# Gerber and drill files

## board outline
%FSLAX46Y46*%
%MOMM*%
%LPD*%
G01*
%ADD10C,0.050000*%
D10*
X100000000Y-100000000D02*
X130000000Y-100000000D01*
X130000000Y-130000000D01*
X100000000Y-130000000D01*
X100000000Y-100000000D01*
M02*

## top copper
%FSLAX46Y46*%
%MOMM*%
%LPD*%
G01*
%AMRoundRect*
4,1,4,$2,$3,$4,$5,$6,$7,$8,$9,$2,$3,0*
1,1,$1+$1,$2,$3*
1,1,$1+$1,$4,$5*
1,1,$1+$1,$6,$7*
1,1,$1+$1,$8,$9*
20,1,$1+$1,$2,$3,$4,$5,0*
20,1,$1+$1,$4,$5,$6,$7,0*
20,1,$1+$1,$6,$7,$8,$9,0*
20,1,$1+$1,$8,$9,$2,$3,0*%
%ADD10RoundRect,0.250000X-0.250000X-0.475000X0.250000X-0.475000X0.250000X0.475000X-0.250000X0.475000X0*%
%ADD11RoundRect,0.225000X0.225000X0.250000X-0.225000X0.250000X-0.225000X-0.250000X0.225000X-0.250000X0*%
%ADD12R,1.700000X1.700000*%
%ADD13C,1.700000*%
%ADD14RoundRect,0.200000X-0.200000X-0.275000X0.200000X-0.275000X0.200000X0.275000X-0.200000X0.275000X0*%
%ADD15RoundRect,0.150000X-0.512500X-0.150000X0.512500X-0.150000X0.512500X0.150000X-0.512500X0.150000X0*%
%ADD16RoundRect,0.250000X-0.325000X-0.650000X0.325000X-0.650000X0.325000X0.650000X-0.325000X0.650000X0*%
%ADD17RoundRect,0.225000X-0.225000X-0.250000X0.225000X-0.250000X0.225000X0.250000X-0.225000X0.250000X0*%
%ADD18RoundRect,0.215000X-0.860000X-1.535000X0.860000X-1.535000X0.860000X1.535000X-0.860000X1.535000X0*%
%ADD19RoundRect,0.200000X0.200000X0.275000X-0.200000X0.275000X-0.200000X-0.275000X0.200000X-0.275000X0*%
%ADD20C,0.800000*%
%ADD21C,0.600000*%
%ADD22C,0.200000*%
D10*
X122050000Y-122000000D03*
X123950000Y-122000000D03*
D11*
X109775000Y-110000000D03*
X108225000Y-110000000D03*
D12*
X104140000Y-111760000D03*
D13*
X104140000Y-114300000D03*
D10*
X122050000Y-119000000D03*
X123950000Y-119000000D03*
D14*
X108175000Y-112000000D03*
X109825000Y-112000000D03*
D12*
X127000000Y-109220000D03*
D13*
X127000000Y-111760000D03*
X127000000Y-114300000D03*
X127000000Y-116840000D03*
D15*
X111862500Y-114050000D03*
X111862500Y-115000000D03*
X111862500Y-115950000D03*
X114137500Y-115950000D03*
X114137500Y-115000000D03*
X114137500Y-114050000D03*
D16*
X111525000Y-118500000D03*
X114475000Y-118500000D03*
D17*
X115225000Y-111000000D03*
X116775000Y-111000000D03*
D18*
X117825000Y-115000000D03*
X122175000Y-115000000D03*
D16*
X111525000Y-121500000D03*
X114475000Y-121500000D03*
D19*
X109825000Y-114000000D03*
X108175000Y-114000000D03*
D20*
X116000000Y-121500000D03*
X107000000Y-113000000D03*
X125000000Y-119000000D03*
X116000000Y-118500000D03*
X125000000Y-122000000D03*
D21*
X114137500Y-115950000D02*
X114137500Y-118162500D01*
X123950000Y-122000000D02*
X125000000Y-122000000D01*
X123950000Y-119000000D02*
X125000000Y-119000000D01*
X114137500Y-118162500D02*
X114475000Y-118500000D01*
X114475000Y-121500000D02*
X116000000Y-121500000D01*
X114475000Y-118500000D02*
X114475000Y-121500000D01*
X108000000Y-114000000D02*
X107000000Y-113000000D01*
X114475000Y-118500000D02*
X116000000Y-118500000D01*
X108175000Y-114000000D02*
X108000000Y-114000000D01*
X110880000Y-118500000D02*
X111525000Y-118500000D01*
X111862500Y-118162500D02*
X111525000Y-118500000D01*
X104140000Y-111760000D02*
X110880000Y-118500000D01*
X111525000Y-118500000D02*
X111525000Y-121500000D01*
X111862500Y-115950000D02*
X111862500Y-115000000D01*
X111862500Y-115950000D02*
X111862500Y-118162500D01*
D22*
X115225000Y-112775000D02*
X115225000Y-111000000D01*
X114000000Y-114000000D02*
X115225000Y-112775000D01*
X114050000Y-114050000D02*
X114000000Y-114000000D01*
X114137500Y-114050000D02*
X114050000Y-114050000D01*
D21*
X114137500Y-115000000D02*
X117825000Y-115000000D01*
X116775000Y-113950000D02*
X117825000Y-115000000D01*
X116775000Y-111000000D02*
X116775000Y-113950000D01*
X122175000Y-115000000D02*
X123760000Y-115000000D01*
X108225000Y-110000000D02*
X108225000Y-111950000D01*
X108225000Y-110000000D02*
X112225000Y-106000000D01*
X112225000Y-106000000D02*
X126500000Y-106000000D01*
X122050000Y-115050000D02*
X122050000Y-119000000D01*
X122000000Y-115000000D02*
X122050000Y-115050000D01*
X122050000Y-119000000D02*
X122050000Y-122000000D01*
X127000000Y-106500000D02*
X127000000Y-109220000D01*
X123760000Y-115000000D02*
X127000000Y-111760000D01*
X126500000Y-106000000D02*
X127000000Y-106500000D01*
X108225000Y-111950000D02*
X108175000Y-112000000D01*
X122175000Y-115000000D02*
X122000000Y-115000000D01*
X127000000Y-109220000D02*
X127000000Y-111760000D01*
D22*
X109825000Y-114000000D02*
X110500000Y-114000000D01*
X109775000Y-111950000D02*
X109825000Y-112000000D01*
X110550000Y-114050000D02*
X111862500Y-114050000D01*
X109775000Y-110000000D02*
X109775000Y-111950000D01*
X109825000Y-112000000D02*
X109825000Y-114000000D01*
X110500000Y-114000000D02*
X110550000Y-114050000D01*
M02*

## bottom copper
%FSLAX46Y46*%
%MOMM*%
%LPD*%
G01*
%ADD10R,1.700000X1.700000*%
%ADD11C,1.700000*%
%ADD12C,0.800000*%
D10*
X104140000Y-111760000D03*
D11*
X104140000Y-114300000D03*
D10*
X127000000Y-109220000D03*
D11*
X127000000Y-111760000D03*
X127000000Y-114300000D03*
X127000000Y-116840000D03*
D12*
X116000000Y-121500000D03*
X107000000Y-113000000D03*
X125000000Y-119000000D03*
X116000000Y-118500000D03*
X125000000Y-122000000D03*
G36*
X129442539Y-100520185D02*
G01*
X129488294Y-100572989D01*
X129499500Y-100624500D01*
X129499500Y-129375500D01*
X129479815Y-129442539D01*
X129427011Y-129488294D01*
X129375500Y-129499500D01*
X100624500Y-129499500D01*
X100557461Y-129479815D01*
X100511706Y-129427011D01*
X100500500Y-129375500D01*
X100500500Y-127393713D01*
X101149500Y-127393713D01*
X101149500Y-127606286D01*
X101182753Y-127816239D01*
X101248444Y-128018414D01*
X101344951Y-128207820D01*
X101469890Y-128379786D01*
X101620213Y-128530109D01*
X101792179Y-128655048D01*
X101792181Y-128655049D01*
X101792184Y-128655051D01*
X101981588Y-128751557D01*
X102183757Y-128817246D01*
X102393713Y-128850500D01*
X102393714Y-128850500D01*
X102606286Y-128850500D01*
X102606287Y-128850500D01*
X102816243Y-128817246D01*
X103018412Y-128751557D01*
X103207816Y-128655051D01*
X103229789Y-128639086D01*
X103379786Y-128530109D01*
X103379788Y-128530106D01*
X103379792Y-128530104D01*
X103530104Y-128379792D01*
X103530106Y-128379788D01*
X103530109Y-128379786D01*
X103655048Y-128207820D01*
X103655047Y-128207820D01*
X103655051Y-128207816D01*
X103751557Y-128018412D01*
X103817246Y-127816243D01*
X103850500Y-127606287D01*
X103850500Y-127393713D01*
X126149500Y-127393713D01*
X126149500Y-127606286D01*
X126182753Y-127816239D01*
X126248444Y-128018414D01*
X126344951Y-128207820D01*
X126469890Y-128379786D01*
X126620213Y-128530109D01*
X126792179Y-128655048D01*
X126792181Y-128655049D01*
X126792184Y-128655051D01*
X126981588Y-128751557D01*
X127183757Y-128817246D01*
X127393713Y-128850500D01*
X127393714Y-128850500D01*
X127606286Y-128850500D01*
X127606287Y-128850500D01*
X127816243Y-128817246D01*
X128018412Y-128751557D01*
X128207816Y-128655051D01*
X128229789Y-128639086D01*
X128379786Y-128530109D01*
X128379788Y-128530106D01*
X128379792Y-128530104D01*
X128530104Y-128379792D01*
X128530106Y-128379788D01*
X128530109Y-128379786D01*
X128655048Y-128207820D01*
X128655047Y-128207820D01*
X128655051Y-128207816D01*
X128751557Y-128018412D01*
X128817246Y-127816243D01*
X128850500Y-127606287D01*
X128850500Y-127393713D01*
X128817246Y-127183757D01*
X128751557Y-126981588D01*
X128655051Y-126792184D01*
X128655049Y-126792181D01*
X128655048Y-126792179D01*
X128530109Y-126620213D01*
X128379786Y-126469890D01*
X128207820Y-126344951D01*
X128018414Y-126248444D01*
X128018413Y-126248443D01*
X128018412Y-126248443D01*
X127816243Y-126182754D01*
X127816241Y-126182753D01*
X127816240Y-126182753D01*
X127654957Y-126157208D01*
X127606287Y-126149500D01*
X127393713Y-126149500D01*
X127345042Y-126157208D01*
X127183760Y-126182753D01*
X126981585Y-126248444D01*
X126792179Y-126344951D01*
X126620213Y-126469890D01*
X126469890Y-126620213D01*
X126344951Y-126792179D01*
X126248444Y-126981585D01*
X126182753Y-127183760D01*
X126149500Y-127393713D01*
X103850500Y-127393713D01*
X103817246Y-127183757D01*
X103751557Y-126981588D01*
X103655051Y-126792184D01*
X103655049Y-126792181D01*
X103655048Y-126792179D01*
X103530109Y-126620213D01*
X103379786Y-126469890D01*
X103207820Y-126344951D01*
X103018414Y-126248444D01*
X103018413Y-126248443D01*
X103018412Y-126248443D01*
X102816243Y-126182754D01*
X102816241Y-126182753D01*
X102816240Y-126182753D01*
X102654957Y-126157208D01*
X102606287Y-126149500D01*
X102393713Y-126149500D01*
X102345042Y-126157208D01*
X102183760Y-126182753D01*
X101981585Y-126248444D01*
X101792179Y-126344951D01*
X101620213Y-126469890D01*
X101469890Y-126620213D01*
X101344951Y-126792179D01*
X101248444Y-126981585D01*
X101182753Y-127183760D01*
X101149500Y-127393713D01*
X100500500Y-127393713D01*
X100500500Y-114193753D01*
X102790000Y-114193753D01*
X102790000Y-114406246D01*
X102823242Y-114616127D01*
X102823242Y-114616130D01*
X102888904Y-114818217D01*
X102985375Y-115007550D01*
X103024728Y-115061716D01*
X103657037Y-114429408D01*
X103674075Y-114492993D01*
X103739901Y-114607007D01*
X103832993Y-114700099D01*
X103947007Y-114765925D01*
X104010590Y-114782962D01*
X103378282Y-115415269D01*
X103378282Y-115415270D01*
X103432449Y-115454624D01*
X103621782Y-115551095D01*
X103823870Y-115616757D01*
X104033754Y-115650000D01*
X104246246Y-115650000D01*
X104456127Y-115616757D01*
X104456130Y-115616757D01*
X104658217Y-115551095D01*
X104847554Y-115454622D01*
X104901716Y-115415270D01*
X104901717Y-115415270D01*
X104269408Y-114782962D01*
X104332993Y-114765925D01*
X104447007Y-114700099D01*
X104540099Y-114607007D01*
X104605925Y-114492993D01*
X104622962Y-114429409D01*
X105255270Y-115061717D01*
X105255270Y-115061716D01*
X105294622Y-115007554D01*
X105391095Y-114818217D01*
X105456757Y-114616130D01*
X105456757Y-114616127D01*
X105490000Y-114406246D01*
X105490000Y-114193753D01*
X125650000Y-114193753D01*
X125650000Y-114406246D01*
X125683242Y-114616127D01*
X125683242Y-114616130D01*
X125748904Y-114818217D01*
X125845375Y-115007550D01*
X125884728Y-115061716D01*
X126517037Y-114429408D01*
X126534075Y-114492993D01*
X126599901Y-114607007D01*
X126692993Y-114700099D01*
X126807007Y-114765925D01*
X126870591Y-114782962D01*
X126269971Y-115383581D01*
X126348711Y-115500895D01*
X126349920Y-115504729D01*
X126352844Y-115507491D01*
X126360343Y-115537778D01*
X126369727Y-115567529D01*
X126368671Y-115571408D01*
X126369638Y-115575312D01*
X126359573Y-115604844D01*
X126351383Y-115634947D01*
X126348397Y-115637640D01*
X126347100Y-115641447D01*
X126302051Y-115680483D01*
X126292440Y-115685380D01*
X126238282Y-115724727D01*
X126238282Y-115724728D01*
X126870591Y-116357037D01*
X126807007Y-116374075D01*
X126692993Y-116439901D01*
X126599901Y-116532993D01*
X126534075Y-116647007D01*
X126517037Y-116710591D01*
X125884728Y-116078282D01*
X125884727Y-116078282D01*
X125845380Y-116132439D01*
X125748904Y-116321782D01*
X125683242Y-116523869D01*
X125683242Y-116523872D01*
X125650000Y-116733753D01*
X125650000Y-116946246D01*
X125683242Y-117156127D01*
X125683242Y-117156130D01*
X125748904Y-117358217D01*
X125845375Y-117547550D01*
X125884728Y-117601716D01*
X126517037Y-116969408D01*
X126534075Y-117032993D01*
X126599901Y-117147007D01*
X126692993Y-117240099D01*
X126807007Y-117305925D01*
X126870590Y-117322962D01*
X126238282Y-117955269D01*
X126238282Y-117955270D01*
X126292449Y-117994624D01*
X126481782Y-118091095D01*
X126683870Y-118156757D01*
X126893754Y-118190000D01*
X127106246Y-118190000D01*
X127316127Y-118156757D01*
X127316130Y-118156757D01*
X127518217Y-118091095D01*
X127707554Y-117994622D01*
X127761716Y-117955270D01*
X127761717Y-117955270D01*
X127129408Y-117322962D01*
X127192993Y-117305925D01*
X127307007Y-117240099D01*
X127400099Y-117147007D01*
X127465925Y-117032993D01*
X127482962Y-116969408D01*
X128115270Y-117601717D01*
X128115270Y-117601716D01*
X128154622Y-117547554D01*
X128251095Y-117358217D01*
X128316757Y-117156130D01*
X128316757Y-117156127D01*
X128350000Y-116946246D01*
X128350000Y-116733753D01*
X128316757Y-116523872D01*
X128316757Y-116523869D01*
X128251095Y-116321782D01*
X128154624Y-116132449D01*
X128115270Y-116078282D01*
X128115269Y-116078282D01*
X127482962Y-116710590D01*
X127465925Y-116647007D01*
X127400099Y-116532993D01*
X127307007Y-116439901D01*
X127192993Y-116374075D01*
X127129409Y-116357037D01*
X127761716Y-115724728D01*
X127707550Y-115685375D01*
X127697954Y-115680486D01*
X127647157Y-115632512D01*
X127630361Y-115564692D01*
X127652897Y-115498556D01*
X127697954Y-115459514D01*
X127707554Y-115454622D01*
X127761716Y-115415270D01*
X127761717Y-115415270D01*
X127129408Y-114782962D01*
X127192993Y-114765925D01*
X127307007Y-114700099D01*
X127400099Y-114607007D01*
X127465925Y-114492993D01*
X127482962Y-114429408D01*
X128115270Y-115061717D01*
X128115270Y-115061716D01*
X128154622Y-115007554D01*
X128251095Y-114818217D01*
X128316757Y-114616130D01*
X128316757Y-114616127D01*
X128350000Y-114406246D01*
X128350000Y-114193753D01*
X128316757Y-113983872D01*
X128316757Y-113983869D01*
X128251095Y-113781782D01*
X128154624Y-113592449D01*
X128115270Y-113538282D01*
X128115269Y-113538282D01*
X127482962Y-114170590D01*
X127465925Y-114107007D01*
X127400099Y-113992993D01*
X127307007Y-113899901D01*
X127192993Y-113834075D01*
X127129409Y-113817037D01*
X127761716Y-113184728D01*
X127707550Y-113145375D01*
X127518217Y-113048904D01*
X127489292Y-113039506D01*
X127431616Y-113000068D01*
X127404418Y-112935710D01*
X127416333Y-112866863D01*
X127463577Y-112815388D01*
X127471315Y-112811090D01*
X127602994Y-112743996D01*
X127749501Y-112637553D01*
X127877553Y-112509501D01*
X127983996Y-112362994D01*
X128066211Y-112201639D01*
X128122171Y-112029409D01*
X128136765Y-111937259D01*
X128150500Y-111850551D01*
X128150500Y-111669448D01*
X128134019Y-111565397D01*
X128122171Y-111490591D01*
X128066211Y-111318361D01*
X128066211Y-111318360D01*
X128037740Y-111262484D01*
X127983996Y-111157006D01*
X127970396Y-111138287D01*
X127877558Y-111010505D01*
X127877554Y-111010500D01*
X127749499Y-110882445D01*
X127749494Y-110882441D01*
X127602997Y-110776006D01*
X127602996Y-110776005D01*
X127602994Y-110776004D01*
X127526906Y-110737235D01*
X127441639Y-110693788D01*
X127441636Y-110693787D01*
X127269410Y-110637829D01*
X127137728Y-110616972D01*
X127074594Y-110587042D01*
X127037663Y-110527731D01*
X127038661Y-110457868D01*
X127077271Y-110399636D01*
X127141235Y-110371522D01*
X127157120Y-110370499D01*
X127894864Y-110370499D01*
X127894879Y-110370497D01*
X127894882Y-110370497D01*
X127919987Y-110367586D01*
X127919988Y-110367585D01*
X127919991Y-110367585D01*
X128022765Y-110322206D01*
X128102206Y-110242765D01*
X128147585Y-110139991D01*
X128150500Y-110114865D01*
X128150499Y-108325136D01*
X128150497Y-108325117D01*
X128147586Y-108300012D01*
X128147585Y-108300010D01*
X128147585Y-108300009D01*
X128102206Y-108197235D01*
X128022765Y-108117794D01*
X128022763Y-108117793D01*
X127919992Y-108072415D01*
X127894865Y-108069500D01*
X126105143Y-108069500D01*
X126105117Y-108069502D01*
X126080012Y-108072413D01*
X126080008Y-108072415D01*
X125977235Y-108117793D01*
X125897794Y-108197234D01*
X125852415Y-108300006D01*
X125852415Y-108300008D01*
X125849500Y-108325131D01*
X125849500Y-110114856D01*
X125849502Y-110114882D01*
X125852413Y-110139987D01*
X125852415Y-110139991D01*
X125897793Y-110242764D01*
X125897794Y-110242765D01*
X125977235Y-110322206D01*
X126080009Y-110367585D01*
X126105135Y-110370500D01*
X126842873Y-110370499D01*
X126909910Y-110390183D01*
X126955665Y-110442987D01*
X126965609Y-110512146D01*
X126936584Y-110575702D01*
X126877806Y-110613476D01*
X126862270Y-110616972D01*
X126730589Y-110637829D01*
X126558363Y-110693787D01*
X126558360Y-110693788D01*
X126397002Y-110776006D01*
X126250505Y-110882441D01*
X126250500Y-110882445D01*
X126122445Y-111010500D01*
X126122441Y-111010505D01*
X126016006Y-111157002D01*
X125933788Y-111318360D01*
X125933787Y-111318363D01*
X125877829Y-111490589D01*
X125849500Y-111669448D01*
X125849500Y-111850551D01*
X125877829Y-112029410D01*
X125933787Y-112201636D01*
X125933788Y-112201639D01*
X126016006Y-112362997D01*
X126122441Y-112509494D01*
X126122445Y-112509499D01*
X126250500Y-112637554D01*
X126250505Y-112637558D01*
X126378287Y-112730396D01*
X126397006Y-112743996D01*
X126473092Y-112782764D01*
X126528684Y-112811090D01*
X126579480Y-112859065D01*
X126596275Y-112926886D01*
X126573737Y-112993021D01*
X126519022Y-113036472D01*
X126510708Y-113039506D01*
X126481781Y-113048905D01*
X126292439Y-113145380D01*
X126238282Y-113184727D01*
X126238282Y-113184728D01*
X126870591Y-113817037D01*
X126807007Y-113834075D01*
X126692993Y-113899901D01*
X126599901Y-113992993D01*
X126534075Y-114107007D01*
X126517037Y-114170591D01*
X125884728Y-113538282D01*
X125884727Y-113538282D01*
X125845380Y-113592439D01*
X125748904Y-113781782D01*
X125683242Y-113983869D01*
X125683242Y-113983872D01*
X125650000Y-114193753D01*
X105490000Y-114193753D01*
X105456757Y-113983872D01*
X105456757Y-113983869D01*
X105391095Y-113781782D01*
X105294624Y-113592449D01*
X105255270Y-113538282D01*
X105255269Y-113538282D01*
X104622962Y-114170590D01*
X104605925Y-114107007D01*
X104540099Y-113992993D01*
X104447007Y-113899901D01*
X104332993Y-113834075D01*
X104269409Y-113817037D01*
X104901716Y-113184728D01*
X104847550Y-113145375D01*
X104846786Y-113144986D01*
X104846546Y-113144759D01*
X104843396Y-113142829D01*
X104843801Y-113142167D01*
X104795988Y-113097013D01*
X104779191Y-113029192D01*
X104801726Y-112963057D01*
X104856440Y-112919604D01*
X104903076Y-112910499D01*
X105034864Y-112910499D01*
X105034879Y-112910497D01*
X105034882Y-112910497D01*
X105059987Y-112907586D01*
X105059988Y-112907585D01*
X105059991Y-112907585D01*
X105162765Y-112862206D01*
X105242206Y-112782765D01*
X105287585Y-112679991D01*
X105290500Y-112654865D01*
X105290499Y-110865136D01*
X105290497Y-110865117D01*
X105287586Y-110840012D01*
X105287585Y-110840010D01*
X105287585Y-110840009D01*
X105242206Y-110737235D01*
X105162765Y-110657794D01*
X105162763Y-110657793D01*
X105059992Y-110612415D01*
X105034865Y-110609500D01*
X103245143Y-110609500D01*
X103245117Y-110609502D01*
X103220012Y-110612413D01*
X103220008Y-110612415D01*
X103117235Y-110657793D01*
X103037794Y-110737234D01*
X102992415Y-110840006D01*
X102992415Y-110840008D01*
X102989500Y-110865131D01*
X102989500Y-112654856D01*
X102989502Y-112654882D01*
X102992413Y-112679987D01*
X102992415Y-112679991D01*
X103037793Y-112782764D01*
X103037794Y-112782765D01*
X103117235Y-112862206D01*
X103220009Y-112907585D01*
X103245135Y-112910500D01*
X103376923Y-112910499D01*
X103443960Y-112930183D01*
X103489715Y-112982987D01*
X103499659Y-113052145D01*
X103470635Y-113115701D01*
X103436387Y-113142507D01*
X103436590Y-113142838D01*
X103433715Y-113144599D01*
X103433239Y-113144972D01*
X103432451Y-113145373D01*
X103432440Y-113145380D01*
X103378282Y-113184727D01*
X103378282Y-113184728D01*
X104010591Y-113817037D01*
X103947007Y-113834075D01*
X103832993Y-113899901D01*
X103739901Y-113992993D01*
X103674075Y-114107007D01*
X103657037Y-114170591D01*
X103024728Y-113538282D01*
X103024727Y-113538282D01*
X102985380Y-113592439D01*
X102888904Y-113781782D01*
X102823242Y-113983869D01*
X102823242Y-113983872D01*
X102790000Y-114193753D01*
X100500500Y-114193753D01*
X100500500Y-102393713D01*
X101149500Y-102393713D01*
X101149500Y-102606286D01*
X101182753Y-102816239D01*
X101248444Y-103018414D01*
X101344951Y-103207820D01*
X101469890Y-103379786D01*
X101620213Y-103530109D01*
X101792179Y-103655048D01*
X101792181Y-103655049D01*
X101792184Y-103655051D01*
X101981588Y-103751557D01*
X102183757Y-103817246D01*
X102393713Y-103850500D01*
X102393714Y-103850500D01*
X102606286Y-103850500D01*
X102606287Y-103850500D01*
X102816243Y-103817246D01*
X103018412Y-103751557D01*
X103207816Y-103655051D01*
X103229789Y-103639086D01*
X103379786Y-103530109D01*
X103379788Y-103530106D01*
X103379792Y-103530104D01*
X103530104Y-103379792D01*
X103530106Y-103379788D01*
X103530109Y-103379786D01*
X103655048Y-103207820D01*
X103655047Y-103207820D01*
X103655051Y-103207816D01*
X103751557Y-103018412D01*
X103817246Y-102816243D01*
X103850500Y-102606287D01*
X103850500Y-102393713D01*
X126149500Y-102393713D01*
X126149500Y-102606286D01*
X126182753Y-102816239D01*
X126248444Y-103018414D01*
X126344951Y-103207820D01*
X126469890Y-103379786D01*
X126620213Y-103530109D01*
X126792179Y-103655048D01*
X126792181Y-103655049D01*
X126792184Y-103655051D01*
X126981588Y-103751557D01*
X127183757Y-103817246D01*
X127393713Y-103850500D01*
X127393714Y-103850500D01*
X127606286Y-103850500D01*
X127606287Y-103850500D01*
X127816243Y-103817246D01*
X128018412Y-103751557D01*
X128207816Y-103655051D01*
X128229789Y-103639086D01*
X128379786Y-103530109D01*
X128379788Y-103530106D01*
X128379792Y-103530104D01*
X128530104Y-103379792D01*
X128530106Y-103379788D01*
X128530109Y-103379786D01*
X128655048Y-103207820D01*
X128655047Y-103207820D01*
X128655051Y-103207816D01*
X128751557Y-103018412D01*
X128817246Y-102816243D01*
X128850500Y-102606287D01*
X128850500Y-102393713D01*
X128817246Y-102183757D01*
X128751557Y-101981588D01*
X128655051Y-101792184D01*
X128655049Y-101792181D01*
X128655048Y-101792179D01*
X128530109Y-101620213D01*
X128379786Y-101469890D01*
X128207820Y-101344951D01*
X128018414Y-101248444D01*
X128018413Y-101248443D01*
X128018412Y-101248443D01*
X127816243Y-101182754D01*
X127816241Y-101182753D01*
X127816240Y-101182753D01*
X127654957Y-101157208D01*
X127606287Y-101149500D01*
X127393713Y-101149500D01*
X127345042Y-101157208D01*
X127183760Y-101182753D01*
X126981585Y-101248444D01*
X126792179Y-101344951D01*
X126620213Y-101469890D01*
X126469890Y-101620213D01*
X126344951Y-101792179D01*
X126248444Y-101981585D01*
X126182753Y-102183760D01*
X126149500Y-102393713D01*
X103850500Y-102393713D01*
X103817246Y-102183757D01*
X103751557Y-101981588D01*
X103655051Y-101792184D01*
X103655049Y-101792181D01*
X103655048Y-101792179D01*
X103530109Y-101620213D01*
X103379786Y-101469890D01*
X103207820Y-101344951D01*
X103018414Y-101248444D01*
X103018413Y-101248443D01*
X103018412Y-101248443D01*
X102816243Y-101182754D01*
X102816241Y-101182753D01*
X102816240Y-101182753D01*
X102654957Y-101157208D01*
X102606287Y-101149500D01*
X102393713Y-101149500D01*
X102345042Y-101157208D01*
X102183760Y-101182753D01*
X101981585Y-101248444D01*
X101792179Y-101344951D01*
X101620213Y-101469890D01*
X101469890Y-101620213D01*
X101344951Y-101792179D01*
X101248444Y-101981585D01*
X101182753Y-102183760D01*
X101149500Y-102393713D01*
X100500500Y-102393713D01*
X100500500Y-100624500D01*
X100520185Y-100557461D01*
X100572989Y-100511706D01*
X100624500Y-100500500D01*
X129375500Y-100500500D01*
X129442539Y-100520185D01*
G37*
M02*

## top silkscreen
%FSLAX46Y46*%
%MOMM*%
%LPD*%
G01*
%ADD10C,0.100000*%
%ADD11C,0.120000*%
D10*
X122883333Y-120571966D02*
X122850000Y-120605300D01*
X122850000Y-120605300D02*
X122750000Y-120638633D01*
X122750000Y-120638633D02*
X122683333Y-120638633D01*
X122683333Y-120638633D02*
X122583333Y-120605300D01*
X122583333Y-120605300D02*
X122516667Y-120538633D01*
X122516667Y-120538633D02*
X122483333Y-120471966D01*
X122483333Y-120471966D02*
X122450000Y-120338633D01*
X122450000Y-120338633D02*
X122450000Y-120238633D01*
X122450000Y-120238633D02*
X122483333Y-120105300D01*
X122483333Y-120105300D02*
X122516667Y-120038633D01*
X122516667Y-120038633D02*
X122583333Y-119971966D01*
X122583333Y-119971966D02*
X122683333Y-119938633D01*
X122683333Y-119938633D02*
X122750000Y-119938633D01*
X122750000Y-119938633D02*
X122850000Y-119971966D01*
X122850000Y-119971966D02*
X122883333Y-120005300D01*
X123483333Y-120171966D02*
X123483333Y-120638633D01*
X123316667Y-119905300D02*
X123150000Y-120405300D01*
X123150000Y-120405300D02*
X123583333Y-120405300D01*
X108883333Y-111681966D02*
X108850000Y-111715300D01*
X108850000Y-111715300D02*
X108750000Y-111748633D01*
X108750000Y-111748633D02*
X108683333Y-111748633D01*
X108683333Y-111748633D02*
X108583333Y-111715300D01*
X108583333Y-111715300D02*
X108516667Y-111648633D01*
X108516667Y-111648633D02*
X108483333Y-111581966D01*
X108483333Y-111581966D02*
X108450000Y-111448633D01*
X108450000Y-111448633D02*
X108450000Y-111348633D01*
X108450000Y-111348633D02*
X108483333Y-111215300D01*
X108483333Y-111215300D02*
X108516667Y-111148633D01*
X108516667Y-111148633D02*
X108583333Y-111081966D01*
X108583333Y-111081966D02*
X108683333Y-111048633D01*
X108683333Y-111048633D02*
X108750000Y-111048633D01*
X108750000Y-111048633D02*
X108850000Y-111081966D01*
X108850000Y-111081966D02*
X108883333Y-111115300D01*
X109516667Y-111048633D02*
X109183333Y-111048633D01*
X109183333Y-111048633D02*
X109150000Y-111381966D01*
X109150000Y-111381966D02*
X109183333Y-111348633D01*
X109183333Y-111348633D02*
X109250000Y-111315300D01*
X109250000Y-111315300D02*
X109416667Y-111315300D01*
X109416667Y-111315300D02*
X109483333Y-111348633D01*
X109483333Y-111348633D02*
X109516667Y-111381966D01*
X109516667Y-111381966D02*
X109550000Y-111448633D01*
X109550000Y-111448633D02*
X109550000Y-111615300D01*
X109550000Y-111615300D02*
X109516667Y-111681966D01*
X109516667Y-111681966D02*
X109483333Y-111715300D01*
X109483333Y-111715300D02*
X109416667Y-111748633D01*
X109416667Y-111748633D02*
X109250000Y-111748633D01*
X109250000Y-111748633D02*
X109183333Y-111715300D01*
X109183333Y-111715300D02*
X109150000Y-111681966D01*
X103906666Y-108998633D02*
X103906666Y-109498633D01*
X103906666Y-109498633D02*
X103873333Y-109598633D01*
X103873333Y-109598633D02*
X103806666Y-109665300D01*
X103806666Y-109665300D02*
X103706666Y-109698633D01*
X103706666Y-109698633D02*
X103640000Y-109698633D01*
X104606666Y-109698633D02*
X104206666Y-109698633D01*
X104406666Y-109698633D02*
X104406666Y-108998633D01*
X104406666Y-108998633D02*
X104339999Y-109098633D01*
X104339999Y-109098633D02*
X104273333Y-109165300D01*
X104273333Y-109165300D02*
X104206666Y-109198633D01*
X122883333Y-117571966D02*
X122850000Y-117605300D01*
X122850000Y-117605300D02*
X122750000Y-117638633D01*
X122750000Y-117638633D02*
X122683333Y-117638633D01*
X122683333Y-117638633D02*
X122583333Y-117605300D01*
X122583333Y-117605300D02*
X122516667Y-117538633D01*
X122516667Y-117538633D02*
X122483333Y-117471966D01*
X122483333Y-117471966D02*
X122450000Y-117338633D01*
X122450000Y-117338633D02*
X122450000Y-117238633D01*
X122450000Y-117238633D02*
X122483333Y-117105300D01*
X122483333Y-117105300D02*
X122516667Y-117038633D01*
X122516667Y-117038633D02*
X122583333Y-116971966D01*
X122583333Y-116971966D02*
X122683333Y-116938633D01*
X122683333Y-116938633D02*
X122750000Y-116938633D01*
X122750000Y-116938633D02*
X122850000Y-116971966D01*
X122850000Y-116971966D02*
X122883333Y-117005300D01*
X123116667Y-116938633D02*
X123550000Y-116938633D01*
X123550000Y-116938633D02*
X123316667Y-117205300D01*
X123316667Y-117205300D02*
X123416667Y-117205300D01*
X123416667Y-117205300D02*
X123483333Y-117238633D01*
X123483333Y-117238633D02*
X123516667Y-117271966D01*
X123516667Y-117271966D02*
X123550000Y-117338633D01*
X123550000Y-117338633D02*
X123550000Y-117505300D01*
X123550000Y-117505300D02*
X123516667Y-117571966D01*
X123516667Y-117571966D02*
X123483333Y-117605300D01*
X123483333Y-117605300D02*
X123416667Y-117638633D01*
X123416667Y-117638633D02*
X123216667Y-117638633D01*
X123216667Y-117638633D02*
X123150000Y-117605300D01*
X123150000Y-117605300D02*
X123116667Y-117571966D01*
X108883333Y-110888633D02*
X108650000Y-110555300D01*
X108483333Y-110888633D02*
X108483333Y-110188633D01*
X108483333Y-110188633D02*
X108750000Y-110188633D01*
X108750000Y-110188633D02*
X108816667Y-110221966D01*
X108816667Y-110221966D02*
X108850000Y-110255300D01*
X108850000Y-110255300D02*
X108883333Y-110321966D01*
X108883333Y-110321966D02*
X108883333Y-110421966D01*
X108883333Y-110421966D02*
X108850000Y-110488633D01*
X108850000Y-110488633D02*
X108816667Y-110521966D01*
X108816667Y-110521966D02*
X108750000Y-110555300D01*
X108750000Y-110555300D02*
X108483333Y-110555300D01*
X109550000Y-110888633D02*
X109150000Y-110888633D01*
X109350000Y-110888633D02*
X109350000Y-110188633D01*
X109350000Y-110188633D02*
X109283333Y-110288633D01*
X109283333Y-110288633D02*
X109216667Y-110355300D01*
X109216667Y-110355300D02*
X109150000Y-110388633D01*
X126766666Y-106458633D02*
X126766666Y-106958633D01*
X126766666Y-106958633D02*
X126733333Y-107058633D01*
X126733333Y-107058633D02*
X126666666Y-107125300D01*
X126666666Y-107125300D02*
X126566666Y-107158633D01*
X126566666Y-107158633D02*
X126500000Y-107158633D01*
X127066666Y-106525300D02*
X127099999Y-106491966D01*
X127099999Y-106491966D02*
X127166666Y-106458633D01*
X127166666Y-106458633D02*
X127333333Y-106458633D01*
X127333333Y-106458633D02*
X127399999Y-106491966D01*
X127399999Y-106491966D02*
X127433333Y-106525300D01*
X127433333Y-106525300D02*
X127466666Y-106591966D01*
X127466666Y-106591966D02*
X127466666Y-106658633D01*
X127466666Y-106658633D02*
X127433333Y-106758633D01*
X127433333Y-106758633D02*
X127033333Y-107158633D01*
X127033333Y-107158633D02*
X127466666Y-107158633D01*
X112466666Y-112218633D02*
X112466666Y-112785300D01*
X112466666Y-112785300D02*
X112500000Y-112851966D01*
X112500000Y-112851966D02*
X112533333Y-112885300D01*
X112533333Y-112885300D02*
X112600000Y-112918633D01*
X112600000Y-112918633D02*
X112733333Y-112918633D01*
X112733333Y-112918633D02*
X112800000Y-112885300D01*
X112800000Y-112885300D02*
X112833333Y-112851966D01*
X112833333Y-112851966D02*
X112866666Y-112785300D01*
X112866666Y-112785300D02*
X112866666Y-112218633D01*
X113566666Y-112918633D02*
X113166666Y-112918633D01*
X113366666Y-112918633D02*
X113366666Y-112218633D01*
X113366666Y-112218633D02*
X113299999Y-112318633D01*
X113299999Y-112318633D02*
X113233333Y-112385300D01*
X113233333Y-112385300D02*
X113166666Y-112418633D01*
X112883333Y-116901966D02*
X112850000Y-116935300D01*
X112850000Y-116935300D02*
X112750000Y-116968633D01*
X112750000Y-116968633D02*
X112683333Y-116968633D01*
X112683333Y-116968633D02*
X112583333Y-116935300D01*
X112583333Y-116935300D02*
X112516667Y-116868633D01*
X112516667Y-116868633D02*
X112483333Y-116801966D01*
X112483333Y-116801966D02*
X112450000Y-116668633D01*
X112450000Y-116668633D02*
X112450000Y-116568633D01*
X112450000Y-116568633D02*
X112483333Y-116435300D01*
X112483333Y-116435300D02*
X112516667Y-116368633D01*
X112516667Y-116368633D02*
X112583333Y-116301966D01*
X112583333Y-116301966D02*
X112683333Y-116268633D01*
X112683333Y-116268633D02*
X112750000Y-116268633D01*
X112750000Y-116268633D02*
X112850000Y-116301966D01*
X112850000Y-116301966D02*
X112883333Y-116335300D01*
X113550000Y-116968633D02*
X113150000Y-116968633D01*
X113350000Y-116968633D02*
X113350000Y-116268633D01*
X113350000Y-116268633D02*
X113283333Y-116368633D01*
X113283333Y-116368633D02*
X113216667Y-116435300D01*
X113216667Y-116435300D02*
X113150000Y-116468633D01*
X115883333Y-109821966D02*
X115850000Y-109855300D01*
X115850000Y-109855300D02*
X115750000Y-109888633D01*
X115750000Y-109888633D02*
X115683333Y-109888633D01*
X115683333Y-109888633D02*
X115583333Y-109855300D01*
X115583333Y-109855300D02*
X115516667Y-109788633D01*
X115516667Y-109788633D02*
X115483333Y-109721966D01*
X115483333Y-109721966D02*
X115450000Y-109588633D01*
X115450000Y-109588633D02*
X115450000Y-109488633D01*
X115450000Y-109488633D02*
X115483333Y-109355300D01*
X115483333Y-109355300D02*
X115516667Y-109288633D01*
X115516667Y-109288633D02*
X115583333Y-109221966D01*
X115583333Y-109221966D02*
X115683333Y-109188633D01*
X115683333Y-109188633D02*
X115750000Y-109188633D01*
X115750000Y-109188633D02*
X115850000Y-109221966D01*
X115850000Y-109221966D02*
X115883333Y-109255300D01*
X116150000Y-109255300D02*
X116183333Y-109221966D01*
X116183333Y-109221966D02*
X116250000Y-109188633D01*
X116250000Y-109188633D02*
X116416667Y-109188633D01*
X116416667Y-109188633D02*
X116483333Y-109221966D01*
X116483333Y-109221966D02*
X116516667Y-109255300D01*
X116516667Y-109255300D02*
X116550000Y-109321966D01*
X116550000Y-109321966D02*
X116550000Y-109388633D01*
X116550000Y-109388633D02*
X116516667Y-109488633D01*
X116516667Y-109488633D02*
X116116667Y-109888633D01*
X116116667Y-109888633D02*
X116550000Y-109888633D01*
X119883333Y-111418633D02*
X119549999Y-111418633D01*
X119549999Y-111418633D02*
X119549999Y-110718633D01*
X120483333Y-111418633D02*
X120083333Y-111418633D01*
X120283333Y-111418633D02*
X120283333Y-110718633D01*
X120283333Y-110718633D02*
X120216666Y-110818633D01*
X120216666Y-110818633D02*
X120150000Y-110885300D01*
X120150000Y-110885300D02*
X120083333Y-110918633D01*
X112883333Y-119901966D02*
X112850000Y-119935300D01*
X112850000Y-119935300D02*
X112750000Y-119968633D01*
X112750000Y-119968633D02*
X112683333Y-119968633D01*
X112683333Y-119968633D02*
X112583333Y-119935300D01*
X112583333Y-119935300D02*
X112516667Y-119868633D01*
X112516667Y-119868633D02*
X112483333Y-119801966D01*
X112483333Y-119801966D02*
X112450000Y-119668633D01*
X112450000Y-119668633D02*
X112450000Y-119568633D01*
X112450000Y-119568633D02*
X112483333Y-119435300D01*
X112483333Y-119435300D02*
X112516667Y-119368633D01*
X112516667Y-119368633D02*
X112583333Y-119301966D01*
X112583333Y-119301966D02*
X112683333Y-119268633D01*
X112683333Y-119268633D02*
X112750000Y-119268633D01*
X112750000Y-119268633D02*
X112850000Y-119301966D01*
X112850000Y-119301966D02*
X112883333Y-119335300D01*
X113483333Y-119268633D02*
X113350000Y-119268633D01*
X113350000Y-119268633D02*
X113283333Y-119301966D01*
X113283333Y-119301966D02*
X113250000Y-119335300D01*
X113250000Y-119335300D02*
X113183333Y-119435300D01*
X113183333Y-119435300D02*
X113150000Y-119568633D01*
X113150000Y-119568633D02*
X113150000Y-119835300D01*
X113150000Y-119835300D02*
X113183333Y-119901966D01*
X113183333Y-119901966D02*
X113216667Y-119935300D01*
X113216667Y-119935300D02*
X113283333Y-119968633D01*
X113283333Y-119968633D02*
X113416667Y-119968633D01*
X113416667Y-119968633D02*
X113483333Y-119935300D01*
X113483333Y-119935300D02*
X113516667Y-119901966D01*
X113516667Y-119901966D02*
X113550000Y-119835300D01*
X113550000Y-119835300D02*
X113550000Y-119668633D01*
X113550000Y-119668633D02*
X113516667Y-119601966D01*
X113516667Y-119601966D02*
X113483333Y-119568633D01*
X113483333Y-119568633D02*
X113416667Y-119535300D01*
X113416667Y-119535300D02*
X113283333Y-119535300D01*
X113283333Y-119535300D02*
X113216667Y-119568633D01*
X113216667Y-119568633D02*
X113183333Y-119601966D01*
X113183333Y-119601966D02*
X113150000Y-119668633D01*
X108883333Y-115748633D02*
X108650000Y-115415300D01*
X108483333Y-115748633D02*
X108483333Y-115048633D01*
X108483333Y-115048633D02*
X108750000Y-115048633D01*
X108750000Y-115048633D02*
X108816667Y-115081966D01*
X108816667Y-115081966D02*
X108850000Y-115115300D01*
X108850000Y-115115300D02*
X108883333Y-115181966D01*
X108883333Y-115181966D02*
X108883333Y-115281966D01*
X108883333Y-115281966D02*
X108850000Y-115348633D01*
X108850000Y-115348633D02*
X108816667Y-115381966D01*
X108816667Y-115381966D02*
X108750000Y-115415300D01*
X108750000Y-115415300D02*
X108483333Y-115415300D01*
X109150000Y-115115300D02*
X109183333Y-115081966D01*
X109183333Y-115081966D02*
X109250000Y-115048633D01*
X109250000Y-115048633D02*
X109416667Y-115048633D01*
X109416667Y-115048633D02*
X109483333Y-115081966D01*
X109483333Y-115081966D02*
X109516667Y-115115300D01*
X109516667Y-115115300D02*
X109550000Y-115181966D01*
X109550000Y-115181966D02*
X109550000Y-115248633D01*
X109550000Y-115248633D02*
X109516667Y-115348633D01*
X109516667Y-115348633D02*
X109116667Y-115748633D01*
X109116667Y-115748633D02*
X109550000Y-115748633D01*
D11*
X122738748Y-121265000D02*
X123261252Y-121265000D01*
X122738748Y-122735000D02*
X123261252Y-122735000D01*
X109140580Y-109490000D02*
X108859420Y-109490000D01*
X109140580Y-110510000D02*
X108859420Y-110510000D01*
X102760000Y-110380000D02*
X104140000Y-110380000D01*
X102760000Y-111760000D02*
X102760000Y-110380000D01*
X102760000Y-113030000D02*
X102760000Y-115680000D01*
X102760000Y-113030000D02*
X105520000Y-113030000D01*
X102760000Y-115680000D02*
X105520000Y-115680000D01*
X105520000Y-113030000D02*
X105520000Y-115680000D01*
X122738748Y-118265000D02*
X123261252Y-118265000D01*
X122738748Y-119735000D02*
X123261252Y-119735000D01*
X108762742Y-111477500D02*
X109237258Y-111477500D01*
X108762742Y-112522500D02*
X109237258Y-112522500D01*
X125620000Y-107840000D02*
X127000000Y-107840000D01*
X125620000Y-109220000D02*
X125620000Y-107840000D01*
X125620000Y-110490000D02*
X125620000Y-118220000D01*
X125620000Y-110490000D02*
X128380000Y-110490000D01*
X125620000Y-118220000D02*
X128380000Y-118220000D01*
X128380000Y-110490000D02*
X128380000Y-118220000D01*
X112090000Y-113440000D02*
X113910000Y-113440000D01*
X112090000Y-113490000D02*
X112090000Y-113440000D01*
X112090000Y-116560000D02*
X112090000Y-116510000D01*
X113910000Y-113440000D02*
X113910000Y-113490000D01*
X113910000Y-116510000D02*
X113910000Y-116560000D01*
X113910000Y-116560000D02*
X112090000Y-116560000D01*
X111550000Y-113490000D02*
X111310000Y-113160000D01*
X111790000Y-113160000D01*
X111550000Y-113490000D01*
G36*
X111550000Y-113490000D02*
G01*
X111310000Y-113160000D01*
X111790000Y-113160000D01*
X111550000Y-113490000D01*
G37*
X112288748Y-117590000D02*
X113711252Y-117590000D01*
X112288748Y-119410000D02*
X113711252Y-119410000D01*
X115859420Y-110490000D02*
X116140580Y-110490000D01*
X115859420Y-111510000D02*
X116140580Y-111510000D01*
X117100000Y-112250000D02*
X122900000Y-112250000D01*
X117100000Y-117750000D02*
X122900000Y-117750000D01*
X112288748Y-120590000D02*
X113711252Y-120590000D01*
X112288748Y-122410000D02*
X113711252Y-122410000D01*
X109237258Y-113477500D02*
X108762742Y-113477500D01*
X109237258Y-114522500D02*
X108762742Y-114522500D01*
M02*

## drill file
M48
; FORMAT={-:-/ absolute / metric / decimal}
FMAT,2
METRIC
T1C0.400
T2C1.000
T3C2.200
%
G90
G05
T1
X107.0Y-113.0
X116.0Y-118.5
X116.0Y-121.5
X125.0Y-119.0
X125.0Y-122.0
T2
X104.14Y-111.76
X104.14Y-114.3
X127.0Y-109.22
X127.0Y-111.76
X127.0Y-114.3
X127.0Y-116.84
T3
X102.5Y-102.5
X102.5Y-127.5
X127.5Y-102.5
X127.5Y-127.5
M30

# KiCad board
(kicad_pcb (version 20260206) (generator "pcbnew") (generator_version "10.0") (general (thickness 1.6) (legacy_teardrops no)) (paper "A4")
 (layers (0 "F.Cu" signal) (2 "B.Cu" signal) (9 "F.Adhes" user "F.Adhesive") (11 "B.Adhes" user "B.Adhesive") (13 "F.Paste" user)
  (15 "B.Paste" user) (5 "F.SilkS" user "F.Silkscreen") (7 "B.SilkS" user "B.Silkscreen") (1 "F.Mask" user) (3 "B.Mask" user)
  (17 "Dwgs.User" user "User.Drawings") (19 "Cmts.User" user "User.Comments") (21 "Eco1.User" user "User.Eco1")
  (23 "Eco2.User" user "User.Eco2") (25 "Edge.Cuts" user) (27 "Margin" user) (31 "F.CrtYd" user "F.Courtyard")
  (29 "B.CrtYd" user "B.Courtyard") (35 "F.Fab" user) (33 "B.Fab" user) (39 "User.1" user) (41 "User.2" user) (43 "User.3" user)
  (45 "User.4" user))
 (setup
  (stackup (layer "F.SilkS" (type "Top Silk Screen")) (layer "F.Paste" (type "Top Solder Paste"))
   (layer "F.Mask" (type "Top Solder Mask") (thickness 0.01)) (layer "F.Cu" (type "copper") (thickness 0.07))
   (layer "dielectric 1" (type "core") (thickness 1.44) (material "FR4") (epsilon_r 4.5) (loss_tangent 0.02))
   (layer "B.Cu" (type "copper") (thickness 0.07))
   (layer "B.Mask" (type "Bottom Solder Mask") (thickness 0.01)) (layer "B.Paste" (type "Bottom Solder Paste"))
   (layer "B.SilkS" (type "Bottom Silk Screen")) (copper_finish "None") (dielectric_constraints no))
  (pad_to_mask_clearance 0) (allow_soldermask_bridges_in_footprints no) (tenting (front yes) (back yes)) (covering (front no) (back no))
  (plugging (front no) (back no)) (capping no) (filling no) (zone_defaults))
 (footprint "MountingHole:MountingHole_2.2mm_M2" (layer "F.Cu") (at 102.5 127.5)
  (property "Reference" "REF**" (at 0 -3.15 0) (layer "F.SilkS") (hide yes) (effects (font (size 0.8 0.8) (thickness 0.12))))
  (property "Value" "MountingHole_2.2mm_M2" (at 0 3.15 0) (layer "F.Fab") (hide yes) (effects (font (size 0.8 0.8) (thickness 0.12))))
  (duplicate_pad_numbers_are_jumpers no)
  (pad "" np_thru_hole circle (at 0 0) (size 2.2 2.2) (drill 2.2) (layers "*.Cu" "*.Mask")))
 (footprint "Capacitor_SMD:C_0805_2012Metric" (layer "F.Cu") (at 123 122)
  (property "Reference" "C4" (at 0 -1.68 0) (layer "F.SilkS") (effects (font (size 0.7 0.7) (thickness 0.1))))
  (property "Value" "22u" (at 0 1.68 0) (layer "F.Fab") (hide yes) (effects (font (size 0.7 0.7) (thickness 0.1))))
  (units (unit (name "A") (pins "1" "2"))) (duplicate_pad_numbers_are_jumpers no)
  (fp_line (start -0.261252 -0.735) (end 0.261252 -0.735) (stroke (width 0.12) (type solid)) (layer "F.SilkS"))
  (fp_line (start -0.261252 0.735) (end 0.261252 0.735) (stroke (width 0.12) (type solid)) (layer "F.SilkS"))
  (pad "1" smd roundrect (at -0.95 0) (size 1 1.45) (layers "F.Cu" "F.Mask" "F.Paste") (roundrect_rratio 0.25) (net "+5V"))
  (pad "2" smd roundrect (at 0.95 0) (size 1 1.45) (layers "F.Cu" "F.Mask" "F.Paste") (roundrect_rratio 0.25) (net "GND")))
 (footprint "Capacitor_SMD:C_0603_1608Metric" (layer "F.Cu") (at 109 110 180)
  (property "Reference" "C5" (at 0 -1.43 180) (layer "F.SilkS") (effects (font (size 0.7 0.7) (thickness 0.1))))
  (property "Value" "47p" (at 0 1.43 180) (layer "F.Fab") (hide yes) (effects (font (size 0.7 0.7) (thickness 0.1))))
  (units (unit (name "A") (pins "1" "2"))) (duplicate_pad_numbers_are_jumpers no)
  (fp_line (start -0.14058 0.51) (end 0.14058 0.51) (stroke (width 0.12) (type solid)) (layer "F.SilkS"))
  (fp_line (start -0.14058 -0.51) (end 0.14058 -0.51) (stroke (width 0.12) (type solid)) (layer "F.SilkS"))
  (pad "1" smd roundrect (at -0.775 0 180) (size 0.9 0.95) (layers "F.Cu" "F.Mask" "F.Paste") (roundrect_rratio 0.25) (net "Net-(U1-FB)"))
  (pad "2" smd roundrect (at 0.775 0 180) (size 0.9 0.95) (layers "F.Cu" "F.Mask" "F.Paste") (roundrect_rratio 0.25) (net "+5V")))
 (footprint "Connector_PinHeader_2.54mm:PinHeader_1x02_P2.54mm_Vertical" (layer "F.Cu") (at 104.14 111.76)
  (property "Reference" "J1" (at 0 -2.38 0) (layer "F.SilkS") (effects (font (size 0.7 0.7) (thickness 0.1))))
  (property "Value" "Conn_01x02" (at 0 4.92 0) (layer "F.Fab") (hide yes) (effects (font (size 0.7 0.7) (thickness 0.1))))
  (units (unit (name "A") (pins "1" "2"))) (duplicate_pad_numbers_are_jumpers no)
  (fp_line (start -1.38 -1.38) (end 0 -1.38) (stroke (width 0.12) (type solid)) (layer "F.SilkS"))
  (fp_line (start -1.38 0) (end -1.38 -1.38) (stroke (width 0.12) (type solid)) (layer "F.SilkS"))
  (fp_line (start -1.38 1.27) (end -1.38 3.92) (stroke (width 0.12) (type solid)) (layer "F.SilkS"))
  (fp_line (start -1.38 1.27) (end 1.38 1.27) (stroke (width 0.12) (type solid)) (layer "F.SilkS"))
  (fp_line (start -1.38 3.92) (end 1.38 3.92) (stroke (width 0.12) (type solid)) (layer "F.SilkS"))
  (fp_line (start 1.38 1.27) (end 1.38 3.92) (stroke (width 0.12) (type solid)) (layer "F.SilkS"))
  (pad "1" thru_hole rect (at 0 0) (size 1.7 1.7) (drill 1) (layers "*.Cu" "*.Mask") (remove_unused_layers no) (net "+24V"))
  (pad "2" thru_hole circle (at 0 2.54) (size 1.7 1.7) (drill 1) (layers "*.Cu" "*.Mask") (remove_unused_layers no) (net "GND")))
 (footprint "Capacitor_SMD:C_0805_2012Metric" (layer "F.Cu") (at 123 119)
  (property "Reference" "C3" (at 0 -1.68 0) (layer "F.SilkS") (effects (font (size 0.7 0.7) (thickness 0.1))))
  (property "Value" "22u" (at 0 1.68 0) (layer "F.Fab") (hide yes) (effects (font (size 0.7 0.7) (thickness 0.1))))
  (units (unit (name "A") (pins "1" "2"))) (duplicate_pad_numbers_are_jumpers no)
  (fp_line (start -0.261252 -0.735) (end 0.261252 -0.735) (stroke (width 0.12) (type solid)) (layer "F.SilkS"))
  (fp_line (start -0.261252 0.735) (end 0.261252 0.735) (stroke (width 0.12) (type solid)) (layer "F.SilkS"))
  (pad "1" smd roundrect (at -0.95 0) (size 1 1.45) (layers "F.Cu" "F.Mask" "F.Paste") (roundrect_rratio 0.25) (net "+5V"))
  (pad "2" smd roundrect (at 0.95 0) (size 1 1.45) (layers "F.Cu" "F.Mask" "F.Paste") (roundrect_rratio 0.25) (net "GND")))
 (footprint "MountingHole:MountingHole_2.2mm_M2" (layer "F.Cu") (at 127.5 127.5)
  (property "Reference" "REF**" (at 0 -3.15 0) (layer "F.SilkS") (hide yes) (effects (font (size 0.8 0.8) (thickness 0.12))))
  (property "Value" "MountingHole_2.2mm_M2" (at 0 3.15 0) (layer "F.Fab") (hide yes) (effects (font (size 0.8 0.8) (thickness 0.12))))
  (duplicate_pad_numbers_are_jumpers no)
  (pad "" np_thru_hole circle (at 0 0) (size 2.2 2.2) (drill 2.2) (layers "*.Cu" "*.Mask")))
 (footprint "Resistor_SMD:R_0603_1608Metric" (layer "F.Cu") (at 109 112)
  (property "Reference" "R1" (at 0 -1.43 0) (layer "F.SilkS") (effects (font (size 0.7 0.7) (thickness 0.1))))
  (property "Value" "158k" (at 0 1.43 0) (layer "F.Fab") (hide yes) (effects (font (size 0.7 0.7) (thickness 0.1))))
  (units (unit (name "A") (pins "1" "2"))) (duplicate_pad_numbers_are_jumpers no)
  (fp_line (start -0.237258 -0.5225) (end 0.237258 -0.5225) (stroke (width 0.12) (type solid)) (layer "F.SilkS"))
  (fp_line (start -0.237258 0.5225) (end 0.237258 0.5225) (stroke (width 0.12) (type solid)) (layer "F.SilkS"))
  (pad "1" smd roundrect (at -0.825 0) (size 0.8 0.95) (layers "F.Cu" "F.Mask" "F.Paste") (roundrect_rratio 0.25) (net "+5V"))
  (pad "2" smd roundrect (at 0.825 0) (size 0.8 0.95) (layers "F.Cu" "F.Mask" "F.Paste") (roundrect_rratio 0.25) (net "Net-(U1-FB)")))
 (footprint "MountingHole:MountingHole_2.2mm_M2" (layer "F.Cu") (at 127.5 102.5)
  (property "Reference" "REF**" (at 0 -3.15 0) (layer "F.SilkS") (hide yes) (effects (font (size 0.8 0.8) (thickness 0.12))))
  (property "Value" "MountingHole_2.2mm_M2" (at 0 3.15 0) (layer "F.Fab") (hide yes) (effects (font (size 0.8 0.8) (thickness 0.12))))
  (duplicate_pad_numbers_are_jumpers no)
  (pad "" np_thru_hole circle (at 0 0) (size 2.2 2.2) (drill 2.2) (layers "*.Cu" "*.Mask")))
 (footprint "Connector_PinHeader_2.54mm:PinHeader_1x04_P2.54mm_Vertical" (layer "F.Cu") (at 127 109.22)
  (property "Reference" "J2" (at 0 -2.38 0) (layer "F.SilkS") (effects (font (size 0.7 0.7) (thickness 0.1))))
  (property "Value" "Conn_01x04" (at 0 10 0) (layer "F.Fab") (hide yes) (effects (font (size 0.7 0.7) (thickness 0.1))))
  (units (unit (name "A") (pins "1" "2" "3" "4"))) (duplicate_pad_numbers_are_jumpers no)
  (fp_line (start -1.38 -1.38) (end 0 -1.38) (stroke (width 0.12) (type solid)) (layer "F.SilkS"))
  (fp_line (start -1.38 0) (end -1.38 -1.38) (stroke (width 0.12) (type solid)) (layer "F.SilkS"))
  (fp_line (start -1.38 1.27) (end -1.38 9) (stroke (width 0.12) (type solid)) (layer "F.SilkS"))
  (fp_line (start -1.38 1.27) (end 1.38 1.27) (stroke (width 0.12) (type solid)) (layer "F.SilkS"))
  (fp_line (start -1.38 9) (end 1.38 9) (stroke (width 0.12) (type solid)) (layer "F.SilkS"))
  (fp_line (start 1.38 1.27) (end 1.38 9) (stroke (width 0.12) (type solid)) (layer "F.SilkS"))
  (pad "1" thru_hole rect (at 0 0) (size 1.7 1.7) (drill 1) (layers "*.Cu" "*.Mask") (remove_unused_layers no) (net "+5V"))
  (pad "2" thru_hole circle (at 0 2.54) (size 1.7 1.7) (drill 1) (layers "*.Cu" "*.Mask") (remove_unused_layers no) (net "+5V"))
  (pad "3" thru_hole circle (at 0 5.08) (size 1.7 1.7) (drill 1) (layers "*.Cu" "*.Mask") (remove_unused_layers no) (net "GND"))
  (pad "4" thru_hole circle (at 0 7.62) (size 1.7 1.7) (drill 1) (layers "*.Cu" "*.Mask") (remove_unused_layers no) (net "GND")))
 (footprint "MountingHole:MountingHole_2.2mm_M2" (layer "F.Cu") (at 102.5 102.5)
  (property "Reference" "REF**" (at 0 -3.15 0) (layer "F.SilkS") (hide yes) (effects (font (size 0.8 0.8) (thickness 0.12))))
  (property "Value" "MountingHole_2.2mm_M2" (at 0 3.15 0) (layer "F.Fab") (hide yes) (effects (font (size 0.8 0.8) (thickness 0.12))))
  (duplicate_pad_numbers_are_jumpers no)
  (pad "" np_thru_hole circle (at 0 0) (size 2.2 2.2) (drill 2.2) (layers "*.Cu" "*.Mask")))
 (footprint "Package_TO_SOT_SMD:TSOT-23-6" (layer "F.Cu") (at 113 115)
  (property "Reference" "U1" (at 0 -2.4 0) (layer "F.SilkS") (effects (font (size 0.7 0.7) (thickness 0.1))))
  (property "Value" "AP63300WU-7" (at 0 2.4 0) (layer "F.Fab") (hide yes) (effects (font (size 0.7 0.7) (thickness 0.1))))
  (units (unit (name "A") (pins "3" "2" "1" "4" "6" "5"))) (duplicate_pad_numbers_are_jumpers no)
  (fp_line (start -0.91 -1.56) (end 0.91 -1.56) (stroke (width 0.12) (type solid)) (layer "F.SilkS"))
  (fp_line (start -0.91 -1.51) (end -0.91 -1.56) (stroke (width 0.12) (type solid)) (layer "F.SilkS"))
  (fp_line (start -0.91 1.56) (end -0.91 1.51) (stroke (width 0.12) (type solid)) (layer "F.SilkS"))
  (fp_line (start 0.91 -1.56) (end 0.91 -1.51) (stroke (width 0.12) (type solid)) (layer "F.SilkS"))
  (fp_line (start 0.91 1.51) (end 0.91 1.56) (stroke (width 0.12) (type solid)) (layer "F.SilkS"))
  (fp_line (start 0.91 1.56) (end -0.91 1.56) (stroke (width 0.12) (type solid)) (layer "F.SilkS"))
  (fp_poly (pts (xy -1.45 -1.51) (xy -1.69 -1.84) (xy -1.21 -1.84)) (stroke (width 0.12) (type solid)) (fill yes) (layer "F.SilkS"))
  (pad "1" smd roundrect (at -1.1375 -0.95) (size 1.325 0.6) (layers "F.Cu" "F.Mask" "F.Paste") (roundrect_rratio 0.25) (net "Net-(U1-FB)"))
  (pad "2" smd roundrect (at -1.1375 0) (size 1.325 0.6) (layers "F.Cu" "F.Mask" "F.Paste") (roundrect_rratio 0.25) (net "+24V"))
  (pad "3" smd roundrect (at -1.1375 0.95) (size 1.325 0.6) (layers "F.Cu" "F.Mask" "F.Paste") (roundrect_rratio 0.25) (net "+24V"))
  (pad "4" smd roundrect (at 1.1375 0.95) (size 1.325 0.6) (layers "F.Cu" "F.Mask" "F.Paste") (roundrect_rratio 0.25) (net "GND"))
  (pad "5" smd roundrect (at 1.1375 0) (size 1.325 0.6) (layers "F.Cu" "F.Mask" "F.Paste") (roundrect_rratio 0.25) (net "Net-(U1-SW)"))
  (pad "6" smd roundrect (at 1.1375 -0.95) (size 1.325 0.6) (layers "F.Cu" "F.Mask" "F.Paste") (roundrect_rratio 0.25) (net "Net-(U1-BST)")))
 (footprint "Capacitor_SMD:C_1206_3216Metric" (layer "F.Cu") (at 113 118.5)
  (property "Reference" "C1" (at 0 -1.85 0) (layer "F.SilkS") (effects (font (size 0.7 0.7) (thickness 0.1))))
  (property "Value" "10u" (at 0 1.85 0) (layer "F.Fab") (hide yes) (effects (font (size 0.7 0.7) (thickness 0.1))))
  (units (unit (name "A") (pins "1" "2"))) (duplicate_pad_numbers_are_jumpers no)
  (fp_line (start -0.711252 -0.91) (end 0.711252 -0.91) (stroke (width 0.12) (type solid)) (layer "F.SilkS"))
  (fp_line (start -0.711252 0.91) (end 0.711252 0.91) (stroke (width 0.12) (type solid)) (layer "F.SilkS"))
  (pad "1" smd roundrect (at -1.475 0) (size 1.15 1.8) (layers "F.Cu" "F.Mask" "F.Paste") (roundrect_rratio 0.217391) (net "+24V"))
  (pad "2" smd roundrect (at 1.475 0) (size 1.15 1.8) (layers "F.Cu" "F.Mask" "F.Paste") (roundrect_rratio 0.217391) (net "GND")))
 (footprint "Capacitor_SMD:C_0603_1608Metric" (layer "F.Cu") (at 116 111)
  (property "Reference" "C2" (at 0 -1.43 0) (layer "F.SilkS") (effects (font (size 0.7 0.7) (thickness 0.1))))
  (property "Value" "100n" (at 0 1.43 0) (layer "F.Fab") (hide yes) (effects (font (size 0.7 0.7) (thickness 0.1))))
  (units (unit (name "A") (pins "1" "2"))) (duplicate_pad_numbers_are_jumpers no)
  (fp_line (start -0.14058 -0.51) (end 0.14058 -0.51) (stroke (width 0.12) (type solid)) (layer "F.SilkS"))
  (fp_line (start -0.14058 0.51) (end 0.14058 0.51) (stroke (width 0.12) (type solid)) (layer "F.SilkS"))
  (pad "1" smd roundrect (at -0.775 0) (size 0.9 0.95) (layers "F.Cu" "F.Mask" "F.Paste") (roundrect_rratio 0.25) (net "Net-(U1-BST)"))
  (pad "2" smd roundrect (at 0.775 0) (size 0.9 0.95) (layers "F.Cu" "F.Mask" "F.Paste") (roundrect_rratio 0.25) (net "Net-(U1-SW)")))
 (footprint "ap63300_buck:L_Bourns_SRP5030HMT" (layer "F.Cu") (at 120 115)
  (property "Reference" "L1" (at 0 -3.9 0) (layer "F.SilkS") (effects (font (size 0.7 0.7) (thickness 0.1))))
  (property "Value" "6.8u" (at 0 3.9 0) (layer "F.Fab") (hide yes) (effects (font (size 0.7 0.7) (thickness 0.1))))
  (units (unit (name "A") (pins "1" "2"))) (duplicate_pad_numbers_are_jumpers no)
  (fp_line (start -2.9 -2.75) (end 2.9 -2.75) (stroke (width 0.12) (type solid)) (layer "F.SilkS"))
  (fp_line (start -2.9 2.75) (end 2.9 2.75) (stroke (width 0.12) (type solid)) (layer "F.SilkS"))
  (pad "1" smd roundrect (at -2.175 0) (size 2.15 3.5) (layers "F.Cu" "F.Mask" "F.Paste") (roundrect_rratio 0.1) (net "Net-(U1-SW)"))
  (pad "2" smd roundrect (at 2.175 0) (size 2.15 3.5) (layers "F.Cu" "F.Mask" "F.Paste") (roundrect_rratio 0.1) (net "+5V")))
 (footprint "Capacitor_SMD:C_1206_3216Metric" (layer "F.Cu") (at 113 121.5)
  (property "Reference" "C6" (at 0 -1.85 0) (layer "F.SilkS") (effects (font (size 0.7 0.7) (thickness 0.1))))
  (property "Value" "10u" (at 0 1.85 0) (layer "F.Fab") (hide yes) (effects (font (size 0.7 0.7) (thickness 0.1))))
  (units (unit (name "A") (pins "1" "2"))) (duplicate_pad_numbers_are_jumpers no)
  (fp_line (start -0.711252 -0.91) (end 0.711252 -0.91) (stroke (width 0.12) (type solid)) (layer "F.SilkS"))
  (fp_line (start -0.711252 0.91) (end 0.711252 0.91) (stroke (width 0.12) (type solid)) (layer "F.SilkS"))
  (pad "1" smd roundrect (at -1.475 0) (size 1.15 1.8) (layers "F.Cu" "F.Mask" "F.Paste") (roundrect_rratio 0.217391) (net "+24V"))
  (pad "2" smd roundrect (at 1.475 0) (size 1.15 1.8) (layers "F.Cu" "F.Mask" "F.Paste") (roundrect_rratio 0.217391) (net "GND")))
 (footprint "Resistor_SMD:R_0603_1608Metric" (layer "F.Cu") (at 109 114 180)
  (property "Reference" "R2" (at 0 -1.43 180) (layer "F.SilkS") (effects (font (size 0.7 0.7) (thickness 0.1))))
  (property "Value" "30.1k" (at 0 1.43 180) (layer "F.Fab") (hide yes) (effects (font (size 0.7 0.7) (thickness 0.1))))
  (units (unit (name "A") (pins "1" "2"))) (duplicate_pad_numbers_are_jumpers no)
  (fp_line (start -0.237258 0.5225) (end 0.237258 0.5225) (stroke (width 0.12) (type solid)) (layer "F.SilkS"))
  (fp_line (start -0.237258 -0.5225) (end 0.237258 -0.5225) (stroke (width 0.12) (type solid)) (layer "F.SilkS"))
  (pad "1" smd roundrect (at -0.825 0 180) (size 0.8 0.95) (layers "F.Cu" "F.Mask" "F.Paste") (roundrect_rratio 0.25) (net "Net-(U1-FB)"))
  (pad "2" smd roundrect (at 0.825 0 180) (size 0.8 0.95) (layers "F.Cu" "F.Mask" "F.Paste") (roundrect_rratio 0.25) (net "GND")))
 (gr_rect (start 100 100) (end 130 130) (stroke (width 0.05) (type solid)) (fill no) (layer "Edge.Cuts"))
 (segment (start 114.1375 115.95) (end 114.1375 118.1625) (width 0.6) (layer "F.Cu") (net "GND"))
 (segment (start 123.95 122) (end 125 122) (width 0.6) (layer "F.Cu") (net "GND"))
 (segment (start 123.95 119) (end 125 119) (width 0.6) (layer "F.Cu") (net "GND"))
 (segment (start 114.1375 118.1625) (end 114.475 118.5) (width 0.6) (layer "F.Cu") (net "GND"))
 (segment (start 114.475 121.5) (end 116 121.5) (width 0.6) (layer "F.Cu") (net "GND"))
 (segment (start 114.475 118.5) (end 114.475 121.5) (width 0.6) (layer "F.Cu") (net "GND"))
 (segment (start 108 114) (end 107 113) (width 0.6) (layer "F.Cu") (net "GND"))
 (segment (start 114.475 118.5) (end 116 118.5) (width 0.6) (layer "F.Cu") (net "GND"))
 (segment (start 108.175 114) (end 108 114) (width 0.6) (layer "F.Cu") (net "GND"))
 (via (at 116 121.5) (size 0.8) (drill 0.4) (layers "F.Cu" "B.Cu") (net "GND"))
 (via (at 107 113) (size 0.8) (drill 0.4) (layers "F.Cu" "B.Cu") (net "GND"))
 (via (at 125 119) (size 0.8) (drill 0.4) (layers "F.Cu" "B.Cu") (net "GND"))
 (via (at 116 118.5) (size 0.8) (drill 0.4) (layers "F.Cu" "B.Cu") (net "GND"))
 (via (at 125 122) (size 0.8) (drill 0.4) (layers "F.Cu" "B.Cu") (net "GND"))
 (segment (start 110.88 118.5) (end 111.525 118.5) (width 0.6) (layer "F.Cu") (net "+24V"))
 (segment (start 111.8625 118.1625) (end 111.525 118.5) (width 0.6) (layer "F.Cu") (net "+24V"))
 (segment (start 104.14 111.76) (end 110.88 118.5) (width 0.6) (layer "F.Cu") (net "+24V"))
 (segment (start 111.525 118.5) (end 111.525 121.5) (width 0.6) (layer "F.Cu") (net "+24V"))
 (segment (start 111.8625 115.95) (end 111.8625 115) (width 0.6) (layer "F.Cu") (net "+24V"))
 (segment (start 111.8625 115.95) (end 111.8625 118.1625) (width 0.6) (layer "F.Cu") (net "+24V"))
 (segment (start 115.225 112.775) (end 115.225 111) (width 0.2) (layer "F.Cu") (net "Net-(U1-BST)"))
 (segment (start 114 114) (end 115.225 112.775) (width 0.2) (layer "F.Cu") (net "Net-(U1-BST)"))
 (segment (start 114.05 114.05) (end 114 114) (width 0.2) (layer "F.Cu") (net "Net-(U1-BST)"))
 (segment (start 114.1375 114.05) (end 114.05 114.05) (width 0.2) (layer "F.Cu") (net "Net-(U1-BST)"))
 (segment (start 114.1375 115) (end 117.825 115) (width 0.6) (layer "F.Cu") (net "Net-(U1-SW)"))
 (segment (start 116.775 113.95) (end 117.825 115) (width 0.6) (layer "F.Cu") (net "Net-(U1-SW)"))
 (segment (start 116.775 111) (end 116.775 113.95) (width 0.6) (layer "F.Cu") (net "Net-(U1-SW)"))
 (segment (start 122.175 115) (end 123.76 115) (width 0.6) (layer "F.Cu") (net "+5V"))
 (segment (start 108.225 110) (end 108.225 111.95) (width 0.6) (layer "F.Cu") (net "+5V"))
 (segment (start 108.225 110) (end 112.225 106) (width 0.6) (layer "F.Cu") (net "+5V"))
 (segment (start 112.225 106) (end 126.5 106) (width 0.6) (layer "F.Cu") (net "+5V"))
 (segment (start 122.05 115.05) (end 122.05 119) (width 0.6) (layer "F.Cu") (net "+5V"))
 (segment (start 122 115) (end 122.05 115.05) (width 0.6) (layer "F.Cu") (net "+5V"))
 (segment (start 122.05 119) (end 122.05 122) (width 0.6) (layer "F.Cu") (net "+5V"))
 (segment (start 127 106.5) (end 127 109.22) (width 0.6) (layer "F.Cu") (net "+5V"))
 (segment (start 123.76 115) (end 127 111.76) (width 0.6) (layer "F.Cu") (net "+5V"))
 (segment (start 126.5 106) (end 127 106.5) (width 0.6) (layer "F.Cu") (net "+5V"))
 (segment (start 108.225 111.95) (end 108.175 112) (width 0.6) (layer "F.Cu") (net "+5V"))
 (segment (start 122.175 115) (end 122 115) (width 0.6) (layer "F.Cu") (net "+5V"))
 (segment (start 127 109.22) (end 127 111.76) (width 0.6) (layer "F.Cu") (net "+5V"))
 (segment (start 109.825 114) (end 110.5 114) (width 0.2) (layer "F.Cu") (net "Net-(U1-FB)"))
 (segment (start 109.775 111.95) (end 109.825 112) (width 0.2) (layer "F.Cu") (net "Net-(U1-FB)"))
 (segment (start 110.55 114.05) (end 111.8625 114.05) (width 0.2) (layer "F.Cu") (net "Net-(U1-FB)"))
 (segment (start 109.775 110) (end 109.775 111.95) (width 0.2) (layer "F.Cu") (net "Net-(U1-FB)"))
 (segment (start 109.825 112) (end 109.825 114) (width 0.2) (layer "F.Cu") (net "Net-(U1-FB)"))
 (segment (start 110.5 114) (end 110.55 114.05) (width 0.2) (layer "F.Cu") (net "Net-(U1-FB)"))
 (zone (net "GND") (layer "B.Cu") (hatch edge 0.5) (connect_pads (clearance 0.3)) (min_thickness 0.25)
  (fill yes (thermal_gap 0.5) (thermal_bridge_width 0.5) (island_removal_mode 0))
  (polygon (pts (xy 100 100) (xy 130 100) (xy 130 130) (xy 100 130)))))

